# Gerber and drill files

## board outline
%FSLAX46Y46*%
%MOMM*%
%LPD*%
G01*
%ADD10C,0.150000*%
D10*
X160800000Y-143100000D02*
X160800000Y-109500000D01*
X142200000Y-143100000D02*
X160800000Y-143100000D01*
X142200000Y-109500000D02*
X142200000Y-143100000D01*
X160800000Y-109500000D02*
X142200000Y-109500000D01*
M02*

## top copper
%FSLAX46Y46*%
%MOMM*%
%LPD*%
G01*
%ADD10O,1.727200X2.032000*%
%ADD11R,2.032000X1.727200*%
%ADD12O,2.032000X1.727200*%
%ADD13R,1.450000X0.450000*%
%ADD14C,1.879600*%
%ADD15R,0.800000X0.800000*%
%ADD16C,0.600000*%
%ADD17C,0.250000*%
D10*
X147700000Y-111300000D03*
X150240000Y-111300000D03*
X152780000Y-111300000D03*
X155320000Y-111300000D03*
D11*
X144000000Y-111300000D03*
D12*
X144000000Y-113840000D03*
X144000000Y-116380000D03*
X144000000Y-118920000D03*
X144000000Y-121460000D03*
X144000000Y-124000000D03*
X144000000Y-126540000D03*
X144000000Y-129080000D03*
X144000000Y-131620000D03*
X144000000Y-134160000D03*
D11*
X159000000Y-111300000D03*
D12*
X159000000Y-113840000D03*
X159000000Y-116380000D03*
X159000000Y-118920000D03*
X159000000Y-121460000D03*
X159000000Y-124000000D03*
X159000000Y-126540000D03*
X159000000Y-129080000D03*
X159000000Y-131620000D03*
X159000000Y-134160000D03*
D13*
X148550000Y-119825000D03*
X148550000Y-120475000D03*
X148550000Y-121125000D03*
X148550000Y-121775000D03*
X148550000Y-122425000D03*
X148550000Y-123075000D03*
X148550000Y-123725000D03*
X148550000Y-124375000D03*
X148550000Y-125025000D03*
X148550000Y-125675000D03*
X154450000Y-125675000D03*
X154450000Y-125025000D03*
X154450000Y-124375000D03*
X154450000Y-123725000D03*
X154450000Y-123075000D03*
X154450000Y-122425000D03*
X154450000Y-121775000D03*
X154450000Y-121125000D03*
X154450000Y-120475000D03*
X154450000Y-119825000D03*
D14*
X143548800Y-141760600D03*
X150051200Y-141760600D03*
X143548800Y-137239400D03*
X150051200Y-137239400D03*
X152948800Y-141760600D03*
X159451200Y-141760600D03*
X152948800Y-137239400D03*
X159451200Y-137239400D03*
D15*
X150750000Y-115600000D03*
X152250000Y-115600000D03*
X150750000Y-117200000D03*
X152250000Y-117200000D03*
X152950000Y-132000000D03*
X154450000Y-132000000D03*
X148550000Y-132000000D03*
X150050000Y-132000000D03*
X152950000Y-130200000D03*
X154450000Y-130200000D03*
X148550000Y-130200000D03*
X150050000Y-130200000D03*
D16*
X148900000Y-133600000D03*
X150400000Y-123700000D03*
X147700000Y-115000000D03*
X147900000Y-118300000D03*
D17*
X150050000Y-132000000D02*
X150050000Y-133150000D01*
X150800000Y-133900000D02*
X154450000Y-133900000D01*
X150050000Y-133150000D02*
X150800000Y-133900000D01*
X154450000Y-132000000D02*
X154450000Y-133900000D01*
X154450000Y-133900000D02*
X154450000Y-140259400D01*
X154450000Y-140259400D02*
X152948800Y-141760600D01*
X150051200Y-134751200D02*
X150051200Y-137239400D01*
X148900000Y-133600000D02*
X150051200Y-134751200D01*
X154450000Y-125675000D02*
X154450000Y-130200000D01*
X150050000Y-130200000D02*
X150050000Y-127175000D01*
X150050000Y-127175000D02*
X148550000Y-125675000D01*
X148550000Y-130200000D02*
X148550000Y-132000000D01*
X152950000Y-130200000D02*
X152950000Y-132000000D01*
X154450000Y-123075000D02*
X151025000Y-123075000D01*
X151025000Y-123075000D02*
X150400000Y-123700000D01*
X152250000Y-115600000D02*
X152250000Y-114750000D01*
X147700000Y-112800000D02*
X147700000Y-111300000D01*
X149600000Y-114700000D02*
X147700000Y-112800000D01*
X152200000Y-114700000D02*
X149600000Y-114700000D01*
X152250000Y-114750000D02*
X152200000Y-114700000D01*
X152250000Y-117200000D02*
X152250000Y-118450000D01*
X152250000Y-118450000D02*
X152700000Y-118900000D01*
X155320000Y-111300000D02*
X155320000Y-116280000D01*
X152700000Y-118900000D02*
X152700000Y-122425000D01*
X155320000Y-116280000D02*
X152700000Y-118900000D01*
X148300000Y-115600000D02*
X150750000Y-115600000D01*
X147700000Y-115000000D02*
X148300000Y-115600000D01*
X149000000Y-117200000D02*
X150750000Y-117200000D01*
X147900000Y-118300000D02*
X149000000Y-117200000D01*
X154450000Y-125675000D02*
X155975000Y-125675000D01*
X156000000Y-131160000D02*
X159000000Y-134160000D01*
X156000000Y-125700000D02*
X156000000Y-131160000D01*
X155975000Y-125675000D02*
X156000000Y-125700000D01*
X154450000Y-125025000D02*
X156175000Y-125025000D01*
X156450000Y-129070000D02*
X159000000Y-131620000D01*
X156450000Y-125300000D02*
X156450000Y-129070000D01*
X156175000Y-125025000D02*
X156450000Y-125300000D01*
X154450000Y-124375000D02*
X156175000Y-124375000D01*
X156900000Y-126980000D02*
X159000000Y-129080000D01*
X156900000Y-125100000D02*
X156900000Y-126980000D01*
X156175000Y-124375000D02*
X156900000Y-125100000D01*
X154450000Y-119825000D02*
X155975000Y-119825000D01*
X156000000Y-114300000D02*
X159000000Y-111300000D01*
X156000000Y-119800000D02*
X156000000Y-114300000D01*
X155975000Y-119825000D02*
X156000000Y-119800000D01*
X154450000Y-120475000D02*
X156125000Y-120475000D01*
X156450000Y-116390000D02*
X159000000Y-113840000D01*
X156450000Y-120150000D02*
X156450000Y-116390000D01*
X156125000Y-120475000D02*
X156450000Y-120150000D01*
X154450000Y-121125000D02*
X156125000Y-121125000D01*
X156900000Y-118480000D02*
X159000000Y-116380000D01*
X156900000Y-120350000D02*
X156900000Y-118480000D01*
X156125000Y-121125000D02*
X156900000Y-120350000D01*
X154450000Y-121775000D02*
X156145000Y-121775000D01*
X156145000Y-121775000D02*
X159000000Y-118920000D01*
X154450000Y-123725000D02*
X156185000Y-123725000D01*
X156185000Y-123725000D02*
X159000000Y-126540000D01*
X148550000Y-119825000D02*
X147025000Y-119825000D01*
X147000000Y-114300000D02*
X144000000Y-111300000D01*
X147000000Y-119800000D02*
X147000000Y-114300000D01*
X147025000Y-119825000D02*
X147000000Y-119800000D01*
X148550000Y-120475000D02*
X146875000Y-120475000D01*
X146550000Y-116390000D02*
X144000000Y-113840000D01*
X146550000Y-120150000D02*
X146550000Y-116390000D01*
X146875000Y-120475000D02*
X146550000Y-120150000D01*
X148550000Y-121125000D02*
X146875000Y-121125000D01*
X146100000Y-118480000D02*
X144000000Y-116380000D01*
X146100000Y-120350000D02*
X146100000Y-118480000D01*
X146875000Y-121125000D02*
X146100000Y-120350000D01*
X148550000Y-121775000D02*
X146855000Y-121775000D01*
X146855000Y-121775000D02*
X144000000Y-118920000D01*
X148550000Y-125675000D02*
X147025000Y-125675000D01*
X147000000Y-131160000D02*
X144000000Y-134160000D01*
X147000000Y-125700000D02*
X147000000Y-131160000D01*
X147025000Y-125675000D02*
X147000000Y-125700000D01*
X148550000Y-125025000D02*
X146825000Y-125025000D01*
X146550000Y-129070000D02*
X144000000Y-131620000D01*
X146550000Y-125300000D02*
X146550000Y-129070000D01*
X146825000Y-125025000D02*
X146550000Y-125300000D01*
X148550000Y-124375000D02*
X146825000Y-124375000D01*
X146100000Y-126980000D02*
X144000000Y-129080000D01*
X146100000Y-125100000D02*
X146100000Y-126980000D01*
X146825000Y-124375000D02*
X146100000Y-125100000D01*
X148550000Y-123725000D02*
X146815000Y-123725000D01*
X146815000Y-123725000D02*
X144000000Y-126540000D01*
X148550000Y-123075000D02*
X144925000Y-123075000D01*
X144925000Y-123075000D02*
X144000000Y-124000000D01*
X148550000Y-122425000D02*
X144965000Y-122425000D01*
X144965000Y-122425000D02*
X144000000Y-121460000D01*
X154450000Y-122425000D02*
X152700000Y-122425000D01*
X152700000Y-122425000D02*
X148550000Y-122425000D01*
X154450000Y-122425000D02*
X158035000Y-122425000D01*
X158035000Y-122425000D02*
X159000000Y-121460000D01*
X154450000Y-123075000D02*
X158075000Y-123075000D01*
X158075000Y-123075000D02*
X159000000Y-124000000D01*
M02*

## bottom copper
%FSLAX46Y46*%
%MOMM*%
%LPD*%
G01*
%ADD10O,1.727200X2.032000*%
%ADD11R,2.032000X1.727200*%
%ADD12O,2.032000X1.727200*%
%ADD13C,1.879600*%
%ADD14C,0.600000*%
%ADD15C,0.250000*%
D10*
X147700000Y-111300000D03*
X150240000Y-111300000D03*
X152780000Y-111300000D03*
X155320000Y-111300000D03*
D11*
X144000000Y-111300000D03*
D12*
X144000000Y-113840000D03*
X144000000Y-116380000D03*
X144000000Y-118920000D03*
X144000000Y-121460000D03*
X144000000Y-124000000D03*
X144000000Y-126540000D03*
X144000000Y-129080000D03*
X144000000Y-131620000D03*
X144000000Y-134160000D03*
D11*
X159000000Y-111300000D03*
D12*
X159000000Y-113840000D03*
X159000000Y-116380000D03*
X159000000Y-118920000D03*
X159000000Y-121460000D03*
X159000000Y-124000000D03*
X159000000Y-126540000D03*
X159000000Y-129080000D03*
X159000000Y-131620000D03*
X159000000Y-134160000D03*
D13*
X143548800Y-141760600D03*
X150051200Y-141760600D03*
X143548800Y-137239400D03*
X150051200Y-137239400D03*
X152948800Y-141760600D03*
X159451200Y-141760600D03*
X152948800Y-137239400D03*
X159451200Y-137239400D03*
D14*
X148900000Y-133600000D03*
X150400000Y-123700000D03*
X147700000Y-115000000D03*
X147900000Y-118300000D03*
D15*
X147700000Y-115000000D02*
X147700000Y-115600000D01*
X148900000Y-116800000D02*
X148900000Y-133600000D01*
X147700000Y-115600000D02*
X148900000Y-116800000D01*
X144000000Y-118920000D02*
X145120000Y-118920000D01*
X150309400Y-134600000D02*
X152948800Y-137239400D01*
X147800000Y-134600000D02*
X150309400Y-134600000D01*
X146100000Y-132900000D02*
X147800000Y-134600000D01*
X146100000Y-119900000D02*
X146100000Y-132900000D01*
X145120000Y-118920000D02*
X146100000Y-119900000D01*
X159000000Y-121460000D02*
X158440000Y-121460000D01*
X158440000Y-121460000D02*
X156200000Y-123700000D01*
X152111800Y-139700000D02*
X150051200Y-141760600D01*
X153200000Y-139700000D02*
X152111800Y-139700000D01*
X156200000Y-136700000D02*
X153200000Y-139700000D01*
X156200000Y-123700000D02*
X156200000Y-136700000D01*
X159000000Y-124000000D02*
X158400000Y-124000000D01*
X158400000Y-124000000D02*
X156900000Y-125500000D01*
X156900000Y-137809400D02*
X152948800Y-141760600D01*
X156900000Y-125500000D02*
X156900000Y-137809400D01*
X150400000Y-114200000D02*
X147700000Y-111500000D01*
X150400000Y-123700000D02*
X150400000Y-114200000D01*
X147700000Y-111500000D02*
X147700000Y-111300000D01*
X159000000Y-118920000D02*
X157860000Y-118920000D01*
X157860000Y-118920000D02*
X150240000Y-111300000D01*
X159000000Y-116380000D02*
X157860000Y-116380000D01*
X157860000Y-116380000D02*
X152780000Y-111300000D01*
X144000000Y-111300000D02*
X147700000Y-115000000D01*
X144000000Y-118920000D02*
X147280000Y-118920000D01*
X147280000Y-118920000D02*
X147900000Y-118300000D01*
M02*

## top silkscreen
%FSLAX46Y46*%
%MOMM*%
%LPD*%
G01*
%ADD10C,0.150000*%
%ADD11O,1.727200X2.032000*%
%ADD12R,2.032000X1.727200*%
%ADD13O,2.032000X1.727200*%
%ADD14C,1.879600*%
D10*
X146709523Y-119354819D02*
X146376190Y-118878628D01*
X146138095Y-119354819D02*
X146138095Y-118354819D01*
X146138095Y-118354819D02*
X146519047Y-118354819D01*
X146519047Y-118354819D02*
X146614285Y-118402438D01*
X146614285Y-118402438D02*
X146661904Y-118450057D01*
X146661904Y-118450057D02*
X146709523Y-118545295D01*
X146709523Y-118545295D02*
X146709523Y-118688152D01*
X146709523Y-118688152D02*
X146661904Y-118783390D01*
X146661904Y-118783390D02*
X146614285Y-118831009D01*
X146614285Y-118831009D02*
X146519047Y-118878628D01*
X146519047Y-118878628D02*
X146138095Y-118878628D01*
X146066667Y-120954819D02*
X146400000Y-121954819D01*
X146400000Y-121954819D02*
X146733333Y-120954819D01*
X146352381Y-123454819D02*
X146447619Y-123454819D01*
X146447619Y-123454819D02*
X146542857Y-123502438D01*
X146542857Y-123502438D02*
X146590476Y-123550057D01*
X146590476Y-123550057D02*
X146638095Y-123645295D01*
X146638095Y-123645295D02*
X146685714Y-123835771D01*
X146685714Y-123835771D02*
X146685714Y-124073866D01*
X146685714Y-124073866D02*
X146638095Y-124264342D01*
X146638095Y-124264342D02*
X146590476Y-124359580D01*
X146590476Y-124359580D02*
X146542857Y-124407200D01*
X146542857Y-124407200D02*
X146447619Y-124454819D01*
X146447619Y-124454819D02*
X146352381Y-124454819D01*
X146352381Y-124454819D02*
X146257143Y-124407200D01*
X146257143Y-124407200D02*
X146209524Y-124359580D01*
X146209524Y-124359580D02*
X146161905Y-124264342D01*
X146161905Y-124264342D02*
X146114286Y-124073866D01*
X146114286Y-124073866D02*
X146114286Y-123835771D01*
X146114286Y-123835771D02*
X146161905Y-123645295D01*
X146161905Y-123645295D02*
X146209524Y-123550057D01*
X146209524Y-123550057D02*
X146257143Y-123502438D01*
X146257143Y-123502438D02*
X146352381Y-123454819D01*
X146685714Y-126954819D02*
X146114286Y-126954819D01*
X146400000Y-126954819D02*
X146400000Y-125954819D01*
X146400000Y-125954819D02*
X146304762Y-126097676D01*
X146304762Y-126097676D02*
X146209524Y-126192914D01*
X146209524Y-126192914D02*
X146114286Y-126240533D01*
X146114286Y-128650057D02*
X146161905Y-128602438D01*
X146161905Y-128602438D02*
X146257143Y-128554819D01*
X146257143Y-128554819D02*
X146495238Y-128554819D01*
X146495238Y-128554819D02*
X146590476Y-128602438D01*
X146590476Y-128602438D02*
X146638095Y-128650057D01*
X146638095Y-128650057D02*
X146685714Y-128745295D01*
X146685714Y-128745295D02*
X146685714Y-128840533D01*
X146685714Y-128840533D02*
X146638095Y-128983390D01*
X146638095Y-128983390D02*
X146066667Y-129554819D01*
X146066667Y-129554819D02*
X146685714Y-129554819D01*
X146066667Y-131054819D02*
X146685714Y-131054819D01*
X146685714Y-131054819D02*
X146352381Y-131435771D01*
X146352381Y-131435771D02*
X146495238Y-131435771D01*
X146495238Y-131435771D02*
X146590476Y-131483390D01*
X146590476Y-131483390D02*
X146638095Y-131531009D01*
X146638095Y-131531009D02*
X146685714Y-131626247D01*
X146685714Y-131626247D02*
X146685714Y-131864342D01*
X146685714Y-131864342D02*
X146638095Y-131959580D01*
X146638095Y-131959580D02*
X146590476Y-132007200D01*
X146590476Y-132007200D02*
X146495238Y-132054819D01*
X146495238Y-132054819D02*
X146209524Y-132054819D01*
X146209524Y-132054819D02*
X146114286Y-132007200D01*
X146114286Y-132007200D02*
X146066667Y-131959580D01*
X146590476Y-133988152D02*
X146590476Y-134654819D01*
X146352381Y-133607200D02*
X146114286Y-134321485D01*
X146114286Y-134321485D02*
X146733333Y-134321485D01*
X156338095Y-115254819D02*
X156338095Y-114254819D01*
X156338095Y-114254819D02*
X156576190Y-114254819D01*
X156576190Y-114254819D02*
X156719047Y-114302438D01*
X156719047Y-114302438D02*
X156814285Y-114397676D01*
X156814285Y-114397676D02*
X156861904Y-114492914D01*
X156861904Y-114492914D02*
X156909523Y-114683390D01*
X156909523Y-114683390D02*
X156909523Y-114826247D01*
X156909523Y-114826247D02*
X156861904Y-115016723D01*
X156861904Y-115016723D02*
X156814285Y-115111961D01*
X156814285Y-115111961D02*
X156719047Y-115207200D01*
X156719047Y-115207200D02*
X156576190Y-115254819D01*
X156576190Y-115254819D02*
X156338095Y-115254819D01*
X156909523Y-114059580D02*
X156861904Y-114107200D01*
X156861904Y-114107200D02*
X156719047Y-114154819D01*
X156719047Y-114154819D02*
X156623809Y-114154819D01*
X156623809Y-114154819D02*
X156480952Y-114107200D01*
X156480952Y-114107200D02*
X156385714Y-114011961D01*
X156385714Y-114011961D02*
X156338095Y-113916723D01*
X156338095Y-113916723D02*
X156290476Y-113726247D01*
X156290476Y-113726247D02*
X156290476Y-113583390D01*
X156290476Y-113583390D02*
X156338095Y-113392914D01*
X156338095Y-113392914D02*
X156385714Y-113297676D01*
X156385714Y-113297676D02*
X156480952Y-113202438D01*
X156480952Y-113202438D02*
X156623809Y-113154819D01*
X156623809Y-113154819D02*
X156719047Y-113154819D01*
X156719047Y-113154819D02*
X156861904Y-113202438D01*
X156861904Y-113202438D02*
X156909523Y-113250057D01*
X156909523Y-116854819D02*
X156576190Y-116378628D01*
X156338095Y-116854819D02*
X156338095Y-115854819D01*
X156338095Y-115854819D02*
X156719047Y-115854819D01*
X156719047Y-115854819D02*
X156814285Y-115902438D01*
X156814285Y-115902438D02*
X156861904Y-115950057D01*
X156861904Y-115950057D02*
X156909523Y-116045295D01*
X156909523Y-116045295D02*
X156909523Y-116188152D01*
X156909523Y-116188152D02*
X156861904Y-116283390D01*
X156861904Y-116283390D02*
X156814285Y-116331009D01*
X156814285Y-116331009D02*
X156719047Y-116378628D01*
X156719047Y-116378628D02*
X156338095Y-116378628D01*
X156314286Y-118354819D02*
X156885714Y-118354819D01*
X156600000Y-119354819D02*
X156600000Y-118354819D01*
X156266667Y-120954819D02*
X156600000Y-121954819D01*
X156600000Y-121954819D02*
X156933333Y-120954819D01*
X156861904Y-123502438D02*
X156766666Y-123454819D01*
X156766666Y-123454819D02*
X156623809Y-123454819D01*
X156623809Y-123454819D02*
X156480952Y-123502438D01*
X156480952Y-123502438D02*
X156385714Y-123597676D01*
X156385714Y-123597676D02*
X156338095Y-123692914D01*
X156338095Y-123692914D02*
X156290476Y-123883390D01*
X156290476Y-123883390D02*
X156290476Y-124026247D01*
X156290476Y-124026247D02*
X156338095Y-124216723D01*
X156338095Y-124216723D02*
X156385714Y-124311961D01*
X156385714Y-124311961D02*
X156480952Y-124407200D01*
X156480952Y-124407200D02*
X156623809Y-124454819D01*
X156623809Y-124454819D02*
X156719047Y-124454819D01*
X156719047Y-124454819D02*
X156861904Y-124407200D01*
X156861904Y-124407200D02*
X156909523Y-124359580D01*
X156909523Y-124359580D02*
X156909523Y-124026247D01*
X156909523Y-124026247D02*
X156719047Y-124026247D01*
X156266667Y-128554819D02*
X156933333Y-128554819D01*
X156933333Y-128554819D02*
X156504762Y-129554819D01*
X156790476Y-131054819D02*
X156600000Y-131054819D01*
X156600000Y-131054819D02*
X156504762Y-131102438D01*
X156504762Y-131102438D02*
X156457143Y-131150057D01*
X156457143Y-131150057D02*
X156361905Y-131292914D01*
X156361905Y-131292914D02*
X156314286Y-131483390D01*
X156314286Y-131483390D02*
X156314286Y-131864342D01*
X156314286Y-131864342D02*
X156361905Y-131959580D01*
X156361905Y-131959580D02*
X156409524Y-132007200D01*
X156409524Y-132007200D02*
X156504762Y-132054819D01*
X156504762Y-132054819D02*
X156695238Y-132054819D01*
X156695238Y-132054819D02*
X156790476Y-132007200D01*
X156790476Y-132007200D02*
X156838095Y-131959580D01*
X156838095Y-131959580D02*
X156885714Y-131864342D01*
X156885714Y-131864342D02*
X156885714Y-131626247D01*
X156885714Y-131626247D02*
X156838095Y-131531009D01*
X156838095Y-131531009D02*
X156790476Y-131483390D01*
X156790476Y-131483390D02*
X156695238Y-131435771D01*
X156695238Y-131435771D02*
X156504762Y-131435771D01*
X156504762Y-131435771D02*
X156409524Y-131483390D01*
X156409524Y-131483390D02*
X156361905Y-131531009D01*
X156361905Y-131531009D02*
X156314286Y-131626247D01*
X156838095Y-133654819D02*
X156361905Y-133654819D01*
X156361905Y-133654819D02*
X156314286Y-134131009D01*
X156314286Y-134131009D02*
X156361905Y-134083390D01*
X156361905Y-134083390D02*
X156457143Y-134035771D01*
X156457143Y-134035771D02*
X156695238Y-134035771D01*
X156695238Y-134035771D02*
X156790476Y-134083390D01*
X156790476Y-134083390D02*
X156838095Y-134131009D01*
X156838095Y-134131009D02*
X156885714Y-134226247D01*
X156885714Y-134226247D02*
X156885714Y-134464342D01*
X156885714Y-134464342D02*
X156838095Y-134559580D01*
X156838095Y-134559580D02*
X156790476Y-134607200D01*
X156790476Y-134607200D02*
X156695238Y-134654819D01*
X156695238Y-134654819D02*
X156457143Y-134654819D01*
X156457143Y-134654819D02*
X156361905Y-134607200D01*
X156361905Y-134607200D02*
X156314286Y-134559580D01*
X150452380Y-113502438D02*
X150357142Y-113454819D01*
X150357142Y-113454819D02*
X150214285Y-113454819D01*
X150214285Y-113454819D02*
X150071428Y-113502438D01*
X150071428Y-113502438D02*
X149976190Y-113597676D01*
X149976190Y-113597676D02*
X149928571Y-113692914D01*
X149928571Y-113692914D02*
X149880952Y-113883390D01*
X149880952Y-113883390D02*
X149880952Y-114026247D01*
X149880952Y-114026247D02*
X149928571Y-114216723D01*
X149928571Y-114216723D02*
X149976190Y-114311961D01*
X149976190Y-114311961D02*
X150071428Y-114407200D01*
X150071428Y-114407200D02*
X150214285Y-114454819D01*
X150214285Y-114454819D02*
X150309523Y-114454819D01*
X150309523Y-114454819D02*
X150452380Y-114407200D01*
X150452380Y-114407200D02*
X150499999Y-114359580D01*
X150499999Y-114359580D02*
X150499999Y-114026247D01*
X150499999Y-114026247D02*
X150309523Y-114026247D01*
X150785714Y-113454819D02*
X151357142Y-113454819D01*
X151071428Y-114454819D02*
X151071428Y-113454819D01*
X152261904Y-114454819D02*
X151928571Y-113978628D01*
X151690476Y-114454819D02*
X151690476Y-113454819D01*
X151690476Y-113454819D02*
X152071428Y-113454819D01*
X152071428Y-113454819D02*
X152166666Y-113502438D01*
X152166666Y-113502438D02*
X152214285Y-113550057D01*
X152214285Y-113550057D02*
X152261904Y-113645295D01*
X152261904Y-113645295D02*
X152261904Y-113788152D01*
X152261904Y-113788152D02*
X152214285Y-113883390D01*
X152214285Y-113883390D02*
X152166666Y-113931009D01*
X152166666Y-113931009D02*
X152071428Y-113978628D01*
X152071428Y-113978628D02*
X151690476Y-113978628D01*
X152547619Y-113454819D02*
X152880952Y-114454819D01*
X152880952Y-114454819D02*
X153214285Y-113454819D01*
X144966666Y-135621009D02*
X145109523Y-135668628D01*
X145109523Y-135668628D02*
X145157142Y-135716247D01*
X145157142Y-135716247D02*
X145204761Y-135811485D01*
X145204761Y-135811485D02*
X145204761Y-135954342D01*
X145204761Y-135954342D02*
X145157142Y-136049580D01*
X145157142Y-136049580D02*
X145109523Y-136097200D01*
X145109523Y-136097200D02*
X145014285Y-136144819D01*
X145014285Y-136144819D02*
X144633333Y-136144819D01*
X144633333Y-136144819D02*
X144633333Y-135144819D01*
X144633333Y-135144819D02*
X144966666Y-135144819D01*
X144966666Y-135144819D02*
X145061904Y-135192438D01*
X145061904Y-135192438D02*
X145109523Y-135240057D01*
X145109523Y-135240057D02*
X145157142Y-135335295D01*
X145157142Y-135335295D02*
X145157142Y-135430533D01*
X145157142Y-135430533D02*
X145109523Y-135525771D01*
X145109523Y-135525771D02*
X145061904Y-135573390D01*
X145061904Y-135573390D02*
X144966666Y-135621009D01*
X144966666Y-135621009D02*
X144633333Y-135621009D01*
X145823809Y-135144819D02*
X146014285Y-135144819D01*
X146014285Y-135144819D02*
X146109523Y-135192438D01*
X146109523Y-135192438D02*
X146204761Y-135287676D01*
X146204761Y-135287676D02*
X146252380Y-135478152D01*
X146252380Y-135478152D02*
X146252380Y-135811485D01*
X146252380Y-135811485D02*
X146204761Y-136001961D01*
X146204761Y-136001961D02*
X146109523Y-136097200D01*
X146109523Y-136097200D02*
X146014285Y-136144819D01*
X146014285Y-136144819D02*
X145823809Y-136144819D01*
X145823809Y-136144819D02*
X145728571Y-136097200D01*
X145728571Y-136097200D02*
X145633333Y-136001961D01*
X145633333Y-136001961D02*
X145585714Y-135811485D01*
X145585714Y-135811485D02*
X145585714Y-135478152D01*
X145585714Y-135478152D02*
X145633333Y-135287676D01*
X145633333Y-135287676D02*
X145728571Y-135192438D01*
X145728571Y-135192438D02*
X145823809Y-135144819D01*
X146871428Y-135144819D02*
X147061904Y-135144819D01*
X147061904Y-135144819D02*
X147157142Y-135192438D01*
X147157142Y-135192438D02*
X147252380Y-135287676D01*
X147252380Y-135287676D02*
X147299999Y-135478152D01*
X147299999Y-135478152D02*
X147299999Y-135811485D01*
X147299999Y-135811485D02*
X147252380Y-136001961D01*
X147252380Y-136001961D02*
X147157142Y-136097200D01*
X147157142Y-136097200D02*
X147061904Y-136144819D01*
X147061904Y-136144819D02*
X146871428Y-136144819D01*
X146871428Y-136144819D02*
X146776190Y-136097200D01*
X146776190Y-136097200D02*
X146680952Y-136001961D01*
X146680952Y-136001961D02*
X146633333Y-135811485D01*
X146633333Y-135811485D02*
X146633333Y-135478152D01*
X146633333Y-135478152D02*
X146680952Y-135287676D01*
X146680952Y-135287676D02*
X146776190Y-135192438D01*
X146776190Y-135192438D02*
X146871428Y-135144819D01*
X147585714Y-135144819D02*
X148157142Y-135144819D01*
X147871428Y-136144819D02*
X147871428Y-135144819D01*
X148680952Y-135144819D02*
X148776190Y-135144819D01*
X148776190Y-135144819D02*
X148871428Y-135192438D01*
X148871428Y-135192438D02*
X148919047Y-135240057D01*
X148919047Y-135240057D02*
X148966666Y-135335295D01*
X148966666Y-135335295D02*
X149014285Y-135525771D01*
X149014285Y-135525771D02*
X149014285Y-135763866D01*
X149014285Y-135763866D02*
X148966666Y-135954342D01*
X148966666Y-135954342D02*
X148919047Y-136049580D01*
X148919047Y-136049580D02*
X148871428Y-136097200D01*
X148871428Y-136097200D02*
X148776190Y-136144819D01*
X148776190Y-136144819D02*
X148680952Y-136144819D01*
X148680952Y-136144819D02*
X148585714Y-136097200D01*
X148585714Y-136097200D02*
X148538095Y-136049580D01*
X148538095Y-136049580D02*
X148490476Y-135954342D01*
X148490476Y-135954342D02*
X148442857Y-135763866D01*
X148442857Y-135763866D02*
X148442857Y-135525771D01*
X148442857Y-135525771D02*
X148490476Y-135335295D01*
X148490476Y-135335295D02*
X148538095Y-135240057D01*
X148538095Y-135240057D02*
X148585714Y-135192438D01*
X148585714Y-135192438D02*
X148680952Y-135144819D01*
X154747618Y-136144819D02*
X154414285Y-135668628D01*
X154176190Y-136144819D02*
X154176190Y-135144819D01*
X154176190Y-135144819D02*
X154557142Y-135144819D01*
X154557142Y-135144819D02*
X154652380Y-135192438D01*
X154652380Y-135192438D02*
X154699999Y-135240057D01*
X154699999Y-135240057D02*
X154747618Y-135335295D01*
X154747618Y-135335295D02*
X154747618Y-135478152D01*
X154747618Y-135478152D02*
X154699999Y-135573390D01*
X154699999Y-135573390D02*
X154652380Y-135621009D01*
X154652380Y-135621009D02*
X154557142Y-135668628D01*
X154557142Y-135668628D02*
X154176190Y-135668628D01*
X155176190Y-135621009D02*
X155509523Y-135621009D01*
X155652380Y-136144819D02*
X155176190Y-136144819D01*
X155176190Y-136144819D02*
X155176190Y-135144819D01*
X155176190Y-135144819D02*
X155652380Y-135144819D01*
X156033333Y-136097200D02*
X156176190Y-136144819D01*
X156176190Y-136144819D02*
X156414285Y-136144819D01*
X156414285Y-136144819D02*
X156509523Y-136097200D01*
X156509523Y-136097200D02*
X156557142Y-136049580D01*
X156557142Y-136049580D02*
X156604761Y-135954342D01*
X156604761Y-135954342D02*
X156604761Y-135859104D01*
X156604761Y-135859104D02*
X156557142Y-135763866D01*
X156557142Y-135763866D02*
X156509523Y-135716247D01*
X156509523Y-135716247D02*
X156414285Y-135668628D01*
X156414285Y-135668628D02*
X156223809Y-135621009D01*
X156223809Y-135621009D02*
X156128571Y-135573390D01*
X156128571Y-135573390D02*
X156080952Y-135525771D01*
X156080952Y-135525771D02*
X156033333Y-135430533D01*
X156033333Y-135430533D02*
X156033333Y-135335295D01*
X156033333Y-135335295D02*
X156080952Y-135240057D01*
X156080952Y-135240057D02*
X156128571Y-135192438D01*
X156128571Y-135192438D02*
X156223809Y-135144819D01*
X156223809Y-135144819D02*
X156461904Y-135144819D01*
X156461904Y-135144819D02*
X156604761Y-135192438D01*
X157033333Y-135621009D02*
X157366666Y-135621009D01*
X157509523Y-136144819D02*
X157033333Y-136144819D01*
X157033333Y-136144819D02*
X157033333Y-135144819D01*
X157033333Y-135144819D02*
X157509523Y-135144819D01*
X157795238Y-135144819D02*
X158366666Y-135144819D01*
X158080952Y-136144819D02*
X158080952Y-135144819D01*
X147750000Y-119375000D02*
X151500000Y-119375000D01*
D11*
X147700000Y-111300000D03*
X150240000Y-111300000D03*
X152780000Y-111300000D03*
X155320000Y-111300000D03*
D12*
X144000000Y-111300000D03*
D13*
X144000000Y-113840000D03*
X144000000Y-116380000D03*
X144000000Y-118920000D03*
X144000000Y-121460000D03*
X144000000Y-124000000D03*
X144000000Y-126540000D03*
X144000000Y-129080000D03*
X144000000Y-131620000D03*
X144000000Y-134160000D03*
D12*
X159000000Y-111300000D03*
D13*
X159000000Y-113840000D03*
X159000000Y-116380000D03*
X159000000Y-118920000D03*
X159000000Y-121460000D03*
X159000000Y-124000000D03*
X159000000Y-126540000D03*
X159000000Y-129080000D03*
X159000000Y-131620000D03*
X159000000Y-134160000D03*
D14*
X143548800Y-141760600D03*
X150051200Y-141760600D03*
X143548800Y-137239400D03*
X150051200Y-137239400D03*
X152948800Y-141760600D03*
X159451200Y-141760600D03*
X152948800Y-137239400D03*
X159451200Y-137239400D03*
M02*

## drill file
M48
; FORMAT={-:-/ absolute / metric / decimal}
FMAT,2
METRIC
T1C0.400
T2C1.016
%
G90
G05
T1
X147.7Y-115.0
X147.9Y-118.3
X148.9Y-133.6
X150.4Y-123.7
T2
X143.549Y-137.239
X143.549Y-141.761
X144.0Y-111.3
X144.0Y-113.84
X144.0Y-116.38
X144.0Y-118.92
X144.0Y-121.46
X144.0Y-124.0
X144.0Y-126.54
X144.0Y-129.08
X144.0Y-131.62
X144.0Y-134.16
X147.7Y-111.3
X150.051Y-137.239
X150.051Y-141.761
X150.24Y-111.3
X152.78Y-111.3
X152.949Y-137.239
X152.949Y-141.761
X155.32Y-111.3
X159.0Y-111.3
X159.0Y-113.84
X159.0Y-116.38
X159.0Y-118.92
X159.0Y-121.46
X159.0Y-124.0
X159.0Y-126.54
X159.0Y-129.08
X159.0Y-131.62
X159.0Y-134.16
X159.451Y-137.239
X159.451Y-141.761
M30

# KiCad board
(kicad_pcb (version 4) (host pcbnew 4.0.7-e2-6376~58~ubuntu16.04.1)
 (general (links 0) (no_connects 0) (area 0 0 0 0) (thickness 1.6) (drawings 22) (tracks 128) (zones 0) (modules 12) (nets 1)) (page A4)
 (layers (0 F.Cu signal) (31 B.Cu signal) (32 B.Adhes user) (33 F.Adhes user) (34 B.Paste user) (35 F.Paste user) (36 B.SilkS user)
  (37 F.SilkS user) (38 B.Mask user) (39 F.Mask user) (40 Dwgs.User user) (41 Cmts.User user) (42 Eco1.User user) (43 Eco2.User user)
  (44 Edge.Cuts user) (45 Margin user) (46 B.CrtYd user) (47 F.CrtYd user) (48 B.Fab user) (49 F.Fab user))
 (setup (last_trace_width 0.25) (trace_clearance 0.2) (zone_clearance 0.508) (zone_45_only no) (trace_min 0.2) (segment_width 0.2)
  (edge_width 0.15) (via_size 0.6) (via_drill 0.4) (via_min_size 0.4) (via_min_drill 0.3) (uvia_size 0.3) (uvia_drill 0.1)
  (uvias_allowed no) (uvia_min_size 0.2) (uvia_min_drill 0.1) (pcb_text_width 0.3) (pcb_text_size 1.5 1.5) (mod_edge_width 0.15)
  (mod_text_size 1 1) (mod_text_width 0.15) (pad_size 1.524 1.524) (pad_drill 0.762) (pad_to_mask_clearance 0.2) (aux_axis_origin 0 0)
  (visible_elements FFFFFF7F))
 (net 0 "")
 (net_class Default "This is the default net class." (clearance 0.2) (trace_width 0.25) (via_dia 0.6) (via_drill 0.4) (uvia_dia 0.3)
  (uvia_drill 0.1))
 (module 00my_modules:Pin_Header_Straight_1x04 (layer F.Cu) (at 147.7 111.3 90)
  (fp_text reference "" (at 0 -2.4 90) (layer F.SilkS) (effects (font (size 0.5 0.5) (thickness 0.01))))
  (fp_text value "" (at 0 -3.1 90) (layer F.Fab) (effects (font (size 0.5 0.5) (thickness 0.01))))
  (pad 1 thru_hole oval (at 0 0 90) (size 2.032 1.7272) (drill 1.016) (layers *.Cu *.Mask F.SilkS))
  (pad 2 thru_hole oval (at 0 2.54 90) (size 2.032 1.7272) (drill 1.016) (layers *.Cu *.Mask F.SilkS))
  (pad 3 thru_hole oval (at 0 5.08 90) (size 2.032 1.7272) (drill 1.016) (layers *.Cu *.Mask F.SilkS))
  (pad 4 thru_hole oval (at 0 7.62 90) (size 2.032 1.7272) (drill 1.016) (layers *.Cu *.Mask F.SilkS)))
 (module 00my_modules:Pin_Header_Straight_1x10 (layer F.Cu) (at 144 111.3)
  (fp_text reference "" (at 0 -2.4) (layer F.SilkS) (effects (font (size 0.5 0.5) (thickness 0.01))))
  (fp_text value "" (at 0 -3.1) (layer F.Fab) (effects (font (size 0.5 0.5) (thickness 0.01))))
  (pad 1 thru_hole rect (at 0 0) (size 2.032 1.7272) (drill 1.016) (layers *.Cu *.Mask F.SilkS))
  (pad 2 thru_hole oval (at 0 2.54) (size 2.032 1.7272) (drill 1.016) (layers *.Cu *.Mask F.SilkS))
  (pad 3 thru_hole oval (at 0 5.08) (size 2.032 1.7272) (drill 1.016) (layers *.Cu *.Mask F.SilkS))
  (pad 4 thru_hole oval (at 0 7.62) (size 2.032 1.7272) (drill 1.016) (layers *.Cu *.Mask F.SilkS))
  (pad 5 thru_hole oval (at 0 10.16) (size 2.032 1.7272) (drill 1.016) (layers *.Cu *.Mask F.SilkS))
  (pad 6 thru_hole oval (at 0 12.7) (size 2.032 1.7272) (drill 1.016) (layers *.Cu *.Mask F.SilkS))
  (pad 7 thru_hole oval (at 0 15.24) (size 2.032 1.7272) (drill 1.016) (layers *.Cu *.Mask F.SilkS))
  (pad 8 thru_hole oval (at 0 17.78) (size 2.032 1.7272) (drill 1.016) (layers *.Cu *.Mask F.SilkS))
  (pad 9 thru_hole oval (at 0 20.32) (size 2.032 1.7272) (drill 1.016) (layers *.Cu *.Mask F.SilkS))
  (pad 10 thru_hole oval (at 0 22.86) (size 2.032 1.7272) (drill 1.016) (layers *.Cu *.Mask F.SilkS)))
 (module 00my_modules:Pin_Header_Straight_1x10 (layer F.Cu) (at 159 111.3)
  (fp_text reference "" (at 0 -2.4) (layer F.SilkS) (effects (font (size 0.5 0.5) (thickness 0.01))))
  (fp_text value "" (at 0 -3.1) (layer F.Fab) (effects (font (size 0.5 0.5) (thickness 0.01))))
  (pad 1 thru_hole rect (at 0 0) (size 2.032 1.7272) (drill 1.016) (layers *.Cu *.Mask F.SilkS))
  (pad 2 thru_hole oval (at 0 2.54) (size 2.032 1.7272) (drill 1.016) (layers *.Cu *.Mask F.SilkS))
  (pad 3 thru_hole oval (at 0 5.08) (size 2.032 1.7272) (drill 1.016) (layers *.Cu *.Mask F.SilkS))
  (pad 4 thru_hole oval (at 0 7.62) (size 2.032 1.7272) (drill 1.016) (layers *.Cu *.Mask F.SilkS))
  (pad 5 thru_hole oval (at 0 10.16) (size 2.032 1.7272) (drill 1.016) (layers *.Cu *.Mask F.SilkS))
  (pad 6 thru_hole oval (at 0 12.7) (size 2.032 1.7272) (drill 1.016) (layers *.Cu *.Mask F.SilkS))
  (pad 7 thru_hole oval (at 0 15.24) (size 2.032 1.7272) (drill 1.016) (layers *.Cu *.Mask F.SilkS))
  (pad 8 thru_hole oval (at 0 17.78) (size 2.032 1.7272) (drill 1.016) (layers *.Cu *.Mask F.SilkS))
  (pad 9 thru_hole oval (at 0 20.32) (size 2.032 1.7272) (drill 1.016) (layers *.Cu *.Mask F.SilkS))
  (pad 10 thru_hole oval (at 0 22.86) (size 2.032 1.7272) (drill 1.016) (layers *.Cu *.Mask F.SilkS)))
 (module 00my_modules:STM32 (layer F.Cu) (at 151.5 122.75)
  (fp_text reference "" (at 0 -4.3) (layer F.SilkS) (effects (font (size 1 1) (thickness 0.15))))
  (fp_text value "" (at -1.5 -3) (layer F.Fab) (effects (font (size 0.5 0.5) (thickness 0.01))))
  (fp_line (start -3.75 -3.375) (end 0 -3.375) (layer F.SilkS) (width 0.15))
  (pad BOOT smd rect (at -2.95 -2.925) (size 1.45 0.45) (layers F.Cu F.Paste F.Mask))
  (pad 2 smd rect (at -2.95 -2.275) (size 1.45 0.45) (layers F.Cu F.Paste F.Mask))
  (pad 3 smd rect (at -2.95 -1.625) (size 1.45 0.45) (layers F.Cu F.Paste F.Mask))
  (pad NRST smd rect (at -2.95 -0.975) (size 1.45 0.45) (layers F.Cu F.Paste F.Mask))
  (pad VCC smd rect (at -2.95 -0.325) (size 1.45 0.45) (layers F.Cu F.Paste F.Mask))
  (pad PA0 smd rect (at -2.95 0.325) (size 1.45 0.45) (layers F.Cu F.Paste F.Mask))
  (pad PA1 smd rect (at -2.95 0.975) (size 1.45 0.45) (layers F.Cu F.Paste F.Mask))
  (pad PA2 smd rect (at -2.95 1.625) (size 1.45 0.45) (layers F.Cu F.Paste F.Mask))
  (pad PA3 smd rect (at -2.95 2.275) (size 1.45 0.45) (layers F.Cu F.Paste F.Mask))
  (pad PA4 smd rect (at -2.95 2.925) (size 1.45 0.45) (layers F.Cu F.Paste F.Mask))
  (pad PA5 smd rect (at 2.95 2.925) (size 1.45 0.45) (layers F.Cu F.Paste F.Mask))
  (pad PA6 smd rect (at 2.95 2.275) (size 1.45 0.45) (layers F.Cu F.Paste F.Mask))
  (pad PA7 smd rect (at 2.95 1.625) (size 1.45 0.45) (layers F.Cu F.Paste F.Mask))
  (pad PB1 smd rect (at 2.95 0.975) (size 1.45 0.45) (layers F.Cu F.Paste F.Mask))
  (pad GND smd rect (at 2.95 0.325) (size 1.45 0.45) (layers F.Cu F.Paste F.Mask))
  (pad VCC smd rect (at 2.95 -0.325) (size 1.45 0.45) (layers F.Cu F.Paste F.Mask))
  (pad TX smd rect (at 2.95 -0.975) (size 1.45 0.45) (layers F.Cu F.Paste F.Mask))
  (pad RX smd rect (at 2.95 -1.625) (size 1.45 0.45) (layers F.Cu F.Paste F.Mask))
  (pad DIO smd rect (at 2.95 -2.275) (size 1.45 0.45) (layers F.Cu F.Paste F.Mask))
  (pad CLK smd rect (at 2.95 -2.925) (size 1.45 0.45) (layers F.Cu F.Paste F.Mask)))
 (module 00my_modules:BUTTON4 (layer F.Cu) (at 146.8 139.5)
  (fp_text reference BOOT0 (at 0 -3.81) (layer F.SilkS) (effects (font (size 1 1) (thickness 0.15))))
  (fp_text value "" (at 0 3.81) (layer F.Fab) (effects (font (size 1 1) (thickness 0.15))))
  (pad 1 thru_hole circle (at -3.2512 2.2606) (size 1.8796 1.8796) (drill 1.016) (layers *.Cu *.Mask F.SilkS))
  (pad 2 thru_hole circle (at 3.2512 2.2606) (size 1.8796 1.8796) (drill 1.016) (layers *.Cu *.Mask F.SilkS))
  (pad 3 thru_hole circle (at -3.2512 -2.2606) (size 1.8796 1.8796) (drill 1.016) (layers *.Cu *.Mask F.SilkS))
  (pad 4 thru_hole circle (at 3.2512 -2.2606) (size 1.8796 1.8796) (drill 1.016) (layers *.Cu *.Mask F.SilkS)))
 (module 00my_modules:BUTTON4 (layer F.Cu) (at 156.2 139.5)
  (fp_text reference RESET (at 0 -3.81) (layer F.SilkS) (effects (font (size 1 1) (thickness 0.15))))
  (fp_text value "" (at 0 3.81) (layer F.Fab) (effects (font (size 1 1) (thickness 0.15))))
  (pad 1 thru_hole circle (at -3.2512 2.2606) (size 1.8796 1.8796) (drill 1.016) (layers *.Cu *.Mask F.SilkS))
  (pad 2 thru_hole circle (at 3.2512 2.2606) (size 1.8796 1.8796) (drill 1.016) (layers *.Cu *.Mask F.SilkS))
  (pad 3 thru_hole circle (at -3.2512 -2.2606) (size 1.8796 1.8796) (drill 1.016) (layers *.Cu *.Mask F.SilkS))
  (pad 4 thru_hole circle (at 3.2512 -2.2606) (size 1.8796 1.8796) (drill 1.016) (layers *.Cu *.Mask F.SilkS)))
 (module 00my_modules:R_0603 (layer F.Cu) (at 151.5 115.6)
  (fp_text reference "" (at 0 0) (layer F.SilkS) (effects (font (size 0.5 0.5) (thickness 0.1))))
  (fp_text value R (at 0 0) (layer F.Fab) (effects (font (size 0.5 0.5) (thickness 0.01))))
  (pad 1 smd rect (at -0.75 0) (size 0.8 0.8) (layers F.Cu F.Paste F.Mask))
  (pad 2 smd rect (at 0.75 0) (size 0.8 0.8) (layers F.Cu F.Paste F.Mask)))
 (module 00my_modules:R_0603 (layer F.Cu) (at 151.5 117.2)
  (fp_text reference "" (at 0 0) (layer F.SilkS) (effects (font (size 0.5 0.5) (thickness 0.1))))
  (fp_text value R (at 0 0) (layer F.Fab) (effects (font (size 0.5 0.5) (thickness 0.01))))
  (pad 1 smd rect (at -0.75 0) (size 0.8 0.8) (layers F.Cu F.Paste F.Mask))
  (pad 2 smd rect (at 0.75 0) (size 0.8 0.8) (layers F.Cu F.Paste F.Mask)))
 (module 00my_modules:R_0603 (layer F.Cu) (at 153.7 132)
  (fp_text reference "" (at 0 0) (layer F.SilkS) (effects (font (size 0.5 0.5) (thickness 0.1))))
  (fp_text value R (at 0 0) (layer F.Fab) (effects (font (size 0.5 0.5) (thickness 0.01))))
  (pad 1 smd rect (at -0.75 0) (size 0.8 0.8) (layers F.Cu F.Paste F.Mask))
  (pad 2 smd rect (at 0.75 0) (size 0.8 0.8) (layers F.Cu F.Paste F.Mask)))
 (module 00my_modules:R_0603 (layer F.Cu) (at 149.3 132)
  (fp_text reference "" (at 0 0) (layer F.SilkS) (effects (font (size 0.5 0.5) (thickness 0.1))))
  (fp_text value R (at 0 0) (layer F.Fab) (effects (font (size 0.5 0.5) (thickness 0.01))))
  (pad 1 smd rect (at -0.75 0) (size 0.8 0.8) (layers F.Cu F.Paste F.Mask))
  (pad 2 smd rect (at 0.75 0) (size 0.8 0.8) (layers F.Cu F.Paste F.Mask)))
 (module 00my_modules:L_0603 (layer F.Cu) (at 153.7 130.2)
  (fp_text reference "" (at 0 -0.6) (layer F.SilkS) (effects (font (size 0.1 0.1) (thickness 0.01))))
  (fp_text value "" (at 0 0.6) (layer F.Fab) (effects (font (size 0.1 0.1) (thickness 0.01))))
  (pad 1 smd rect (at -0.75 0) (size 0.8 0.8) (layers F.Cu F.Paste F.Mask))
  (pad 2 smd rect (at 0.75 0) (size 0.8 0.8) (layers F.Cu F.Paste F.Mask)))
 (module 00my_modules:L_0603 (layer F.Cu) (at 149.3 130.2)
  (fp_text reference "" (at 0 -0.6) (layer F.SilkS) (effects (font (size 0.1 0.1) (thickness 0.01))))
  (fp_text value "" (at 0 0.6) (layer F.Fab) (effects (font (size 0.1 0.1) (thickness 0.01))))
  (pad 1 smd rect (at -0.75 0) (size 0.8 0.8) (layers F.Cu F.Paste F.Mask))
  (pad 2 smd rect (at 0.75 0) (size 0.8 0.8) (layers F.Cu F.Paste F.Mask)))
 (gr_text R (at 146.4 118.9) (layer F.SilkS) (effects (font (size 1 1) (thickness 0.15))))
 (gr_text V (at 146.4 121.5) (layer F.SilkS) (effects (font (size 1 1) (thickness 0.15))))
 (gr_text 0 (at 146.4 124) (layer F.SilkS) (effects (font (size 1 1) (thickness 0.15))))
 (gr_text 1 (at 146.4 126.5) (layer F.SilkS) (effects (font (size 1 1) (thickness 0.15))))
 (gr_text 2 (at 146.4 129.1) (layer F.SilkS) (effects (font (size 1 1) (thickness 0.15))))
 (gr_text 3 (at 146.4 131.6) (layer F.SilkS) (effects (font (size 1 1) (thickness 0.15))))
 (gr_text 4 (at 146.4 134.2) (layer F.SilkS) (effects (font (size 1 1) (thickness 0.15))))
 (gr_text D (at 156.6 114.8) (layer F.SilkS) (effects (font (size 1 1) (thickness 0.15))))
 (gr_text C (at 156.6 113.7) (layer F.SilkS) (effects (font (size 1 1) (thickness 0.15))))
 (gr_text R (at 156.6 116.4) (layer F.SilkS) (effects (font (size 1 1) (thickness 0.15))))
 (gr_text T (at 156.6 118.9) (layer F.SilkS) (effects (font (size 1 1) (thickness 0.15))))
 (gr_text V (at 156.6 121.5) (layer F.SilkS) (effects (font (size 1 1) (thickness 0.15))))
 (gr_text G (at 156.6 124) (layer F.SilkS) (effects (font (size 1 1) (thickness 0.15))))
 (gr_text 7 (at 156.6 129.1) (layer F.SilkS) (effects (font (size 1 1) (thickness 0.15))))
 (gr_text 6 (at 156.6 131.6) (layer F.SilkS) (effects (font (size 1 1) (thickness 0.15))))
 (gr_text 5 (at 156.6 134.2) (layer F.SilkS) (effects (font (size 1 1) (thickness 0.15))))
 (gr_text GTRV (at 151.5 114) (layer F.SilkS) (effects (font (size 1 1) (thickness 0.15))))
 (gr_line (start 160.8 143.1) (end 160.8 109.5) (angle 90) (layer Edge.Cuts) (width 0.15))
 (gr_line (start 142.2 143.1) (end 160.8 143.1) (angle 90) (layer Edge.Cuts) (width 0.15))
 (gr_line (start 142.2 109.5) (end 142.2 143.1) (angle 90) (layer Edge.Cuts) (width 0.15))
 (gr_line (start 160.8 109.5) (end 142.2 109.5) (angle 90) (layer Edge.Cuts) (width 0.15))
 (segment (start 150.05 132) (end 150.05 133.15) (width 0.25) (layer F.Cu) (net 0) (status 400000))
 (segment (start 150.8 133.9) (end 154.45 133.9) (width 0.25) (layer F.Cu) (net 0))
 (segment (start 150.05 133.15) (end 150.8 133.9) (width 0.25) (layer F.Cu) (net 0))
 (segment (start 154.45 132) (end 154.45 133.9) (width 0.25) (layer F.Cu) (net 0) (status 400000))
 (segment (start 154.45 133.9) (end 154.45 140.2594) (width 0.25) (layer F.Cu) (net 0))
 (segment (start 154.45 140.2594) (end 152.9488 141.7606) (width 0.25) (layer F.Cu) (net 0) (status 800000))
 (segment (start 147.7 115) (end 147.7 115.6) (width 0.25) (layer B.Cu) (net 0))
 (segment (start 150.0512 134.7512) (end 150.0512 137.2394) (width 0.25) (layer F.Cu) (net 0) (status 800000))
 (segment (start 148.9 133.6) (end 150.0512 134.7512) (width 0.25) (layer F.Cu) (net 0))
 (via (at 148.9 133.6) (size 0.6) (drill 0.4) (layers F.Cu B.Cu) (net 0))
 (segment (start 148.9 116.8) (end 148.9 133.6) (width 0.25) (layer B.Cu) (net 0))
 (segment (start 147.7 115.6) (end 148.9 116.8) (width 0.25) (layer B.Cu) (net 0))
 (segment (start 144 118.92) (end 145.12 118.92) (width 0.25) (layer B.Cu) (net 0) (status 400000))
 (segment (start 150.3094 134.6) (end 152.9488 137.2394) (width 0.25) (layer B.Cu) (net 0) (status 800000))
 (segment (start 147.8 134.6) (end 150.3094 134.6) (width 0.25) (layer B.Cu) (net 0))
 (segment (start 146.1 132.9) (end 147.8 134.6) (width 0.25) (layer B.Cu) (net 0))
 (segment (start 146.1 119.9) (end 146.1 132.9) (width 0.25) (layer B.Cu) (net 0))
 (segment (start 145.12 118.92) (end 146.1 119.9) (width 0.25) (layer B.Cu) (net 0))
 (segment (start 159 121.46) (end 158.44 121.46) (width 0.25) (layer B.Cu) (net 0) (status C00000))
 (segment (start 158.44 121.46) (end 156.2 123.7) (width 0.25) (layer B.Cu) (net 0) (status 400000))
 (segment (start 152.1118 139.7) (end 150.0512 141.7606) (width 0.25) (layer B.Cu) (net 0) (status 800000))
 (segment (start 153.2 139.7) (end 152.1118 139.7) (width 0.25) (layer B.Cu) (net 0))
 (segment (start 156.2 136.7) (end 153.2 139.7) (width 0.25) (layer B.Cu) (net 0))
 (segment (start 156.2 123.7) (end 156.2 136.7) (width 0.25) (layer B.Cu) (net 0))
 (segment (start 159 124) (end 158.4 124) (width 0.25) (layer B.Cu) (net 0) (status C00000))
 (segment (start 158.4 124) (end 156.9 125.5) (width 0.25) (layer B.Cu) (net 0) (status 400000))
 (segment (start 156.9 137.8094) (end 152.9488 141.7606) (width 0.25) (layer B.Cu) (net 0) (status 800000))
 (segment (start 156.9 125.5) (end 156.9 137.8094) (width 0.25) (layer B.Cu) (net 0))
 (segment (start 154.45 125.675) (end 154.45 130.2) (width 0.25) (layer F.Cu) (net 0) (status C00000))
 (segment (start 150.05 130.2) (end 150.05 127.175) (width 0.25) (layer F.Cu) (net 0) (status 400000))
 (segment (start 150.05 127.175) (end 148.55 125.675) (width 0.25) (layer F.Cu) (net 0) (status 800000))
 (segment (start 148.55 130.2) (end 148.55 132) (width 0.25) (layer F.Cu) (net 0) (status C00000))
 (segment (start 152.95 130.2) (end 152.95 132) (width 0.25) (layer F.Cu) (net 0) (status C00000))
 (segment (start 154.45 123.075) (end 151.025 123.075) (width 0.25) (layer F.Cu) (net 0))
 (segment (start 150.4 114.2) (end 147.7 111.5) (width 0.25) (layer B.Cu) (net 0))
 (segment (start 150.4 123.7) (end 150.4 114.2) (width 0.25) (layer B.Cu) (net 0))
 (via (at 150.4 123.7) (size 0.6) (drill 0.4) (layers F.Cu B.Cu) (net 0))
 (segment (start 151.025 123.075) (end 150.4 123.7) (width 0.25) (layer F.Cu) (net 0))
 (segment (start 147.7 111.5) (end 147.7 111.3) (width 0.25) (layer B.Cu) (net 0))
 (segment (start 152.25 115.6) (end 152.25 114.75) (width 0.25) (layer F.Cu) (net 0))
 (segment (start 147.7 112.8) (end 147.7 111.3) (width 0.25) (layer F.Cu) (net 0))
 (segment (start 149.6 114.7) (end 147.7 112.8) (width 0.25) (layer F.Cu) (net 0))
 (segment (start 152.2 114.7) (end 149.6 114.7) (width 0.25) (layer F.Cu) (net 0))
 (segment (start 152.25 114.75) (end 152.2 114.7) (width 0.25) (layer F.Cu) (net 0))
 (segment (start 152.25 117.2) (end 152.25 118.45) (width 0.25) (layer F.Cu) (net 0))
 (segment (start 152.25 118.45) (end 152.7 118.9) (width 0.25) (layer F.Cu) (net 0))
 (segment (start 155.32 111.3) (end 155.32 116.28) (width 0.25) (layer F.Cu) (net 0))
 (segment (start 152.7 118.9) (end 152.7 122.425) (width 0.25) (layer F.Cu) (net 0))
 (segment (start 155.32 116.28) (end 152.7 118.9) (width 0.25) (layer F.Cu) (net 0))
 (segment (start 159 118.92) (end 157.86 118.92) (width 0.25) (layer B.Cu) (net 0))
 (segment (start 157.86 118.92) (end 150.24 111.3) (width 0.25) (layer B.Cu) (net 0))
 (segment (start 159 116.38) (end 157.86 116.38) (width 0.25) (layer B.Cu) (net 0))
 (segment (start 157.86 116.38) (end 152.78 111.3) (width 0.25) (layer B.Cu) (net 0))
 (segment (start 144 111.3) (end 147.7 115) (width 0.25) (layer B.Cu) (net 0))
 (segment (start 148.3 115.6) (end 150.75 115.6) (width 0.25) (layer F.Cu) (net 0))
 (segment (start 147.7 115) (end 148.3 115.6) (width 0.25) (layer F.Cu) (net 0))
 (via (at 147.7 115) (size 0.6) (drill 0.4) (layers F.Cu B.Cu) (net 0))
 (segment (start 144 118.92) (end 147.28 118.92) (width 0.25) (layer B.Cu) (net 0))
 (segment (start 149 117.2) (end 150.75 117.2) (width 0.25) (layer F.Cu) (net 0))
 (segment (start 147.9 118.3) (end 149 117.2) (width 0.25) (layer F.Cu) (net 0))
 (via (at 147.9 118.3) (size 0.6) (drill 0.4) (layers F.Cu B.Cu) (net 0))
 (segment (start 147.28 118.92) (end 147.9 118.3) (width 0.25) (layer B.Cu) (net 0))
 (segment (start 154.45 125.675) (end 155.975 125.675) (width 0.25) (layer F.Cu) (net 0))
 (segment (start 156 131.16) (end 159 134.16) (width 0.25) (layer F.Cu) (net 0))
 (segment (start 156 125.7) (end 156 131.16) (width 0.25) (layer F.Cu) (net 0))
 (segment (start 155.975 125.675) (end 156 125.7) (width 0.25) (layer F.Cu) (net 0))
 (segment (start 154.45 125.025) (end 156.175 125.025) (width 0.25) (layer F.Cu) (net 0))
 (segment (start 156.45 129.07) (end 159 131.62) (width 0.25) (layer F.Cu) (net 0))
 (segment (start 156.45 125.3) (end 156.45 129.07) (width 0.25) (layer F.Cu) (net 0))
 (segment (start 156.175 125.025) (end 156.45 125.3) (width 0.25) (layer F.Cu) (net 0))
 (segment (start 154.45 124.375) (end 156.175 124.375) (width 0.25) (layer F.Cu) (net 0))
 (segment (start 156.9 126.98) (end 159 129.08) (width 0.25) (layer F.Cu) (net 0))
 (segment (start 156.9 125.1) (end 156.9 126.98) (width 0.25) (layer F.Cu) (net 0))
 (segment (start 156.175 124.375) (end 156.9 125.1) (width 0.25) (layer F.Cu) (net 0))
 (segment (start 154.45 119.825) (end 155.975 119.825) (width 0.25) (layer F.Cu) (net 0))
 (segment (start 156 114.3) (end 159 111.3) (width 0.25) (layer F.Cu) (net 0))
 (segment (start 156 119.8) (end 156 114.3) (width 0.25) (layer F.Cu) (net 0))
 (segment (start 155.975 119.825) (end 156 119.8) (width 0.25) (layer F.Cu) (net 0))
 (segment (start 154.45 120.475) (end 156.125 120.475) (width 0.25) (layer F.Cu) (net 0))
 (segment (start 156.45 116.39) (end 159 113.84) (width 0.25) (layer F.Cu) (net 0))
 (segment (start 156.45 120.15) (end 156.45 116.39) (width 0.25) (layer F.Cu) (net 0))
 (segment (start 156.125 120.475) (end 156.45 120.15) (width 0.25) (layer F.Cu) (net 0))
 (segment (start 154.45 121.125) (end 156.125 121.125) (width 0.25) (layer F.Cu) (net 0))
 (segment (start 156.9 118.48) (end 159 116.38) (width 0.25) (layer F.Cu) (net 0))
 (segment (start 156.9 120.35) (end 156.9 118.48) (width 0.25) (layer F.Cu) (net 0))
 (segment (start 156.125 121.125) (end 156.9 120.35) (width 0.25) (layer F.Cu) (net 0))
 (segment (start 154.45 121.775) (end 156.145 121.775) (width 0.25) (layer F.Cu) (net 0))
 (segment (start 156.145 121.775) (end 159 118.92) (width 0.25) (layer F.Cu) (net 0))
 (segment (start 154.45 123.725) (end 156.185 123.725) (width 0.25) (layer F.Cu) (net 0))
 (segment (start 156.185 123.725) (end 159 126.54) (width 0.25) (layer F.Cu) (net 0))
 (segment (start 148.55 119.825) (end 147.025 119.825) (width 0.25) (layer F.Cu) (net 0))
 (segment (start 147 114.3) (end 144 111.3) (width 0.25) (layer F.Cu) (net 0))
 (segment (start 147 119.8) (end 147 114.3) (width 0.25) (layer F.Cu) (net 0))
 (segment (start 147.025 119.825) (end 147 119.8) (width 0.25) (layer F.Cu) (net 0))
 (segment (start 148.55 120.475) (end 146.875 120.475) (width 0.25) (layer F.Cu) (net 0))
 (segment (start 146.55 116.39) (end 144 113.84) (width 0.25) (layer F.Cu) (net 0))
 (segment (start 146.55 120.15) (end 146.55 116.39) (width 0.25) (layer F.Cu) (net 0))
 (segment (start 146.875 120.475) (end 146.55 120.15) (width 0.25) (layer F.Cu) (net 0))
 (segment (start 148.55 121.125) (end 146.875 121.125) (width 0.25) (layer F.Cu) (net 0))
 (segment (start 146.1 118.48) (end 144 116.38) (width 0.25) (layer F.Cu) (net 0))
 (segment (start 146.1 120.35) (end 146.1 118.48) (width 0.25) (layer F.Cu) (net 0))
 (segment (start 146.875 121.125) (end 146.1 120.35) (width 0.25) (layer F.Cu) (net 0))
 (segment (start 148.55 121.775) (end 146.855 121.775) (width 0.25) (layer F.Cu) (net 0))
 (segment (start 146.855 121.775) (end 144 118.92) (width 0.25) (layer F.Cu) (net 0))
 (segment (start 148.55 125.675) (end 147.025 125.675) (width 0.25) (layer F.Cu) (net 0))
 (segment (start 147 131.16) (end 144 134.16) (width 0.25) (layer F.Cu) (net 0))
 (segment (start 147 125.7) (end 147 131.16) (width 0.25) (layer F.Cu) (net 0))
 (segment (start 147.025 125.675) (end 147 125.7) (width 0.25) (layer F.Cu) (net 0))
 (segment (start 148.55 125.025) (end 146.825 125.025) (width 0.25) (layer F.Cu) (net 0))
 (segment (start 146.55 129.07) (end 144 131.62) (width 0.25) (layer F.Cu) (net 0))
 (segment (start 146.55 125.3) (end 146.55 129.07) (width 0.25) (layer F.Cu) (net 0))
 (segment (start 146.825 125.025) (end 146.55 125.3) (width 0.25) (layer F.Cu) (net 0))
 (segment (start 148.55 124.375) (end 146.825 124.375) (width 0.25) (layer F.Cu) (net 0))
 (segment (start 146.1 126.98) (end 144 129.08) (width 0.25) (layer F.Cu) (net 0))
 (segment (start 146.1 125.1) (end 146.1 126.98) (width 0.25) (layer F.Cu) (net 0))
 (segment (start 146.825 124.375) (end 146.1 125.1) (width 0.25) (layer F.Cu) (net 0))
 (segment (start 148.55 123.725) (end 146.815 123.725) (width 0.25) (layer F.Cu) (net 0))
 (segment (start 146.815 123.725) (end 144 126.54) (width 0.25) (layer F.Cu) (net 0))
 (segment (start 148.55 123.075) (end 144.925 123.075) (width 0.25) (layer F.Cu) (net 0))
 (segment (start 144.925 123.075) (end 144 124) (width 0.25) (layer F.Cu) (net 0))
 (segment (start 148.55 122.425) (end 144.965 122.425) (width 0.25) (layer F.Cu) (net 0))
 (segment (start 144.965 122.425) (end 144 121.46) (width 0.25) (layer F.Cu) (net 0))
 (segment (start 154.45 122.425) (end 152.7 122.425) (width 0.25) (layer F.Cu) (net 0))
 (segment (start 152.7 122.425) (end 148.55 122.425) (width 0.25) (layer F.Cu) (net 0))
 (segment (start 154.45 122.425) (end 158.035 122.425) (width 0.25) (layer F.Cu) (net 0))
 (segment (start 158.035 122.425) (end 159 121.46) (width 0.25) (layer F.Cu) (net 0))
 (segment (start 154.45 123.075) (end 158.075 123.075) (width 0.25) (layer F.Cu) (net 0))
 (segment (start 158.075 123.075) (end 159 124) (width 0.25) (layer F.Cu) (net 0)))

